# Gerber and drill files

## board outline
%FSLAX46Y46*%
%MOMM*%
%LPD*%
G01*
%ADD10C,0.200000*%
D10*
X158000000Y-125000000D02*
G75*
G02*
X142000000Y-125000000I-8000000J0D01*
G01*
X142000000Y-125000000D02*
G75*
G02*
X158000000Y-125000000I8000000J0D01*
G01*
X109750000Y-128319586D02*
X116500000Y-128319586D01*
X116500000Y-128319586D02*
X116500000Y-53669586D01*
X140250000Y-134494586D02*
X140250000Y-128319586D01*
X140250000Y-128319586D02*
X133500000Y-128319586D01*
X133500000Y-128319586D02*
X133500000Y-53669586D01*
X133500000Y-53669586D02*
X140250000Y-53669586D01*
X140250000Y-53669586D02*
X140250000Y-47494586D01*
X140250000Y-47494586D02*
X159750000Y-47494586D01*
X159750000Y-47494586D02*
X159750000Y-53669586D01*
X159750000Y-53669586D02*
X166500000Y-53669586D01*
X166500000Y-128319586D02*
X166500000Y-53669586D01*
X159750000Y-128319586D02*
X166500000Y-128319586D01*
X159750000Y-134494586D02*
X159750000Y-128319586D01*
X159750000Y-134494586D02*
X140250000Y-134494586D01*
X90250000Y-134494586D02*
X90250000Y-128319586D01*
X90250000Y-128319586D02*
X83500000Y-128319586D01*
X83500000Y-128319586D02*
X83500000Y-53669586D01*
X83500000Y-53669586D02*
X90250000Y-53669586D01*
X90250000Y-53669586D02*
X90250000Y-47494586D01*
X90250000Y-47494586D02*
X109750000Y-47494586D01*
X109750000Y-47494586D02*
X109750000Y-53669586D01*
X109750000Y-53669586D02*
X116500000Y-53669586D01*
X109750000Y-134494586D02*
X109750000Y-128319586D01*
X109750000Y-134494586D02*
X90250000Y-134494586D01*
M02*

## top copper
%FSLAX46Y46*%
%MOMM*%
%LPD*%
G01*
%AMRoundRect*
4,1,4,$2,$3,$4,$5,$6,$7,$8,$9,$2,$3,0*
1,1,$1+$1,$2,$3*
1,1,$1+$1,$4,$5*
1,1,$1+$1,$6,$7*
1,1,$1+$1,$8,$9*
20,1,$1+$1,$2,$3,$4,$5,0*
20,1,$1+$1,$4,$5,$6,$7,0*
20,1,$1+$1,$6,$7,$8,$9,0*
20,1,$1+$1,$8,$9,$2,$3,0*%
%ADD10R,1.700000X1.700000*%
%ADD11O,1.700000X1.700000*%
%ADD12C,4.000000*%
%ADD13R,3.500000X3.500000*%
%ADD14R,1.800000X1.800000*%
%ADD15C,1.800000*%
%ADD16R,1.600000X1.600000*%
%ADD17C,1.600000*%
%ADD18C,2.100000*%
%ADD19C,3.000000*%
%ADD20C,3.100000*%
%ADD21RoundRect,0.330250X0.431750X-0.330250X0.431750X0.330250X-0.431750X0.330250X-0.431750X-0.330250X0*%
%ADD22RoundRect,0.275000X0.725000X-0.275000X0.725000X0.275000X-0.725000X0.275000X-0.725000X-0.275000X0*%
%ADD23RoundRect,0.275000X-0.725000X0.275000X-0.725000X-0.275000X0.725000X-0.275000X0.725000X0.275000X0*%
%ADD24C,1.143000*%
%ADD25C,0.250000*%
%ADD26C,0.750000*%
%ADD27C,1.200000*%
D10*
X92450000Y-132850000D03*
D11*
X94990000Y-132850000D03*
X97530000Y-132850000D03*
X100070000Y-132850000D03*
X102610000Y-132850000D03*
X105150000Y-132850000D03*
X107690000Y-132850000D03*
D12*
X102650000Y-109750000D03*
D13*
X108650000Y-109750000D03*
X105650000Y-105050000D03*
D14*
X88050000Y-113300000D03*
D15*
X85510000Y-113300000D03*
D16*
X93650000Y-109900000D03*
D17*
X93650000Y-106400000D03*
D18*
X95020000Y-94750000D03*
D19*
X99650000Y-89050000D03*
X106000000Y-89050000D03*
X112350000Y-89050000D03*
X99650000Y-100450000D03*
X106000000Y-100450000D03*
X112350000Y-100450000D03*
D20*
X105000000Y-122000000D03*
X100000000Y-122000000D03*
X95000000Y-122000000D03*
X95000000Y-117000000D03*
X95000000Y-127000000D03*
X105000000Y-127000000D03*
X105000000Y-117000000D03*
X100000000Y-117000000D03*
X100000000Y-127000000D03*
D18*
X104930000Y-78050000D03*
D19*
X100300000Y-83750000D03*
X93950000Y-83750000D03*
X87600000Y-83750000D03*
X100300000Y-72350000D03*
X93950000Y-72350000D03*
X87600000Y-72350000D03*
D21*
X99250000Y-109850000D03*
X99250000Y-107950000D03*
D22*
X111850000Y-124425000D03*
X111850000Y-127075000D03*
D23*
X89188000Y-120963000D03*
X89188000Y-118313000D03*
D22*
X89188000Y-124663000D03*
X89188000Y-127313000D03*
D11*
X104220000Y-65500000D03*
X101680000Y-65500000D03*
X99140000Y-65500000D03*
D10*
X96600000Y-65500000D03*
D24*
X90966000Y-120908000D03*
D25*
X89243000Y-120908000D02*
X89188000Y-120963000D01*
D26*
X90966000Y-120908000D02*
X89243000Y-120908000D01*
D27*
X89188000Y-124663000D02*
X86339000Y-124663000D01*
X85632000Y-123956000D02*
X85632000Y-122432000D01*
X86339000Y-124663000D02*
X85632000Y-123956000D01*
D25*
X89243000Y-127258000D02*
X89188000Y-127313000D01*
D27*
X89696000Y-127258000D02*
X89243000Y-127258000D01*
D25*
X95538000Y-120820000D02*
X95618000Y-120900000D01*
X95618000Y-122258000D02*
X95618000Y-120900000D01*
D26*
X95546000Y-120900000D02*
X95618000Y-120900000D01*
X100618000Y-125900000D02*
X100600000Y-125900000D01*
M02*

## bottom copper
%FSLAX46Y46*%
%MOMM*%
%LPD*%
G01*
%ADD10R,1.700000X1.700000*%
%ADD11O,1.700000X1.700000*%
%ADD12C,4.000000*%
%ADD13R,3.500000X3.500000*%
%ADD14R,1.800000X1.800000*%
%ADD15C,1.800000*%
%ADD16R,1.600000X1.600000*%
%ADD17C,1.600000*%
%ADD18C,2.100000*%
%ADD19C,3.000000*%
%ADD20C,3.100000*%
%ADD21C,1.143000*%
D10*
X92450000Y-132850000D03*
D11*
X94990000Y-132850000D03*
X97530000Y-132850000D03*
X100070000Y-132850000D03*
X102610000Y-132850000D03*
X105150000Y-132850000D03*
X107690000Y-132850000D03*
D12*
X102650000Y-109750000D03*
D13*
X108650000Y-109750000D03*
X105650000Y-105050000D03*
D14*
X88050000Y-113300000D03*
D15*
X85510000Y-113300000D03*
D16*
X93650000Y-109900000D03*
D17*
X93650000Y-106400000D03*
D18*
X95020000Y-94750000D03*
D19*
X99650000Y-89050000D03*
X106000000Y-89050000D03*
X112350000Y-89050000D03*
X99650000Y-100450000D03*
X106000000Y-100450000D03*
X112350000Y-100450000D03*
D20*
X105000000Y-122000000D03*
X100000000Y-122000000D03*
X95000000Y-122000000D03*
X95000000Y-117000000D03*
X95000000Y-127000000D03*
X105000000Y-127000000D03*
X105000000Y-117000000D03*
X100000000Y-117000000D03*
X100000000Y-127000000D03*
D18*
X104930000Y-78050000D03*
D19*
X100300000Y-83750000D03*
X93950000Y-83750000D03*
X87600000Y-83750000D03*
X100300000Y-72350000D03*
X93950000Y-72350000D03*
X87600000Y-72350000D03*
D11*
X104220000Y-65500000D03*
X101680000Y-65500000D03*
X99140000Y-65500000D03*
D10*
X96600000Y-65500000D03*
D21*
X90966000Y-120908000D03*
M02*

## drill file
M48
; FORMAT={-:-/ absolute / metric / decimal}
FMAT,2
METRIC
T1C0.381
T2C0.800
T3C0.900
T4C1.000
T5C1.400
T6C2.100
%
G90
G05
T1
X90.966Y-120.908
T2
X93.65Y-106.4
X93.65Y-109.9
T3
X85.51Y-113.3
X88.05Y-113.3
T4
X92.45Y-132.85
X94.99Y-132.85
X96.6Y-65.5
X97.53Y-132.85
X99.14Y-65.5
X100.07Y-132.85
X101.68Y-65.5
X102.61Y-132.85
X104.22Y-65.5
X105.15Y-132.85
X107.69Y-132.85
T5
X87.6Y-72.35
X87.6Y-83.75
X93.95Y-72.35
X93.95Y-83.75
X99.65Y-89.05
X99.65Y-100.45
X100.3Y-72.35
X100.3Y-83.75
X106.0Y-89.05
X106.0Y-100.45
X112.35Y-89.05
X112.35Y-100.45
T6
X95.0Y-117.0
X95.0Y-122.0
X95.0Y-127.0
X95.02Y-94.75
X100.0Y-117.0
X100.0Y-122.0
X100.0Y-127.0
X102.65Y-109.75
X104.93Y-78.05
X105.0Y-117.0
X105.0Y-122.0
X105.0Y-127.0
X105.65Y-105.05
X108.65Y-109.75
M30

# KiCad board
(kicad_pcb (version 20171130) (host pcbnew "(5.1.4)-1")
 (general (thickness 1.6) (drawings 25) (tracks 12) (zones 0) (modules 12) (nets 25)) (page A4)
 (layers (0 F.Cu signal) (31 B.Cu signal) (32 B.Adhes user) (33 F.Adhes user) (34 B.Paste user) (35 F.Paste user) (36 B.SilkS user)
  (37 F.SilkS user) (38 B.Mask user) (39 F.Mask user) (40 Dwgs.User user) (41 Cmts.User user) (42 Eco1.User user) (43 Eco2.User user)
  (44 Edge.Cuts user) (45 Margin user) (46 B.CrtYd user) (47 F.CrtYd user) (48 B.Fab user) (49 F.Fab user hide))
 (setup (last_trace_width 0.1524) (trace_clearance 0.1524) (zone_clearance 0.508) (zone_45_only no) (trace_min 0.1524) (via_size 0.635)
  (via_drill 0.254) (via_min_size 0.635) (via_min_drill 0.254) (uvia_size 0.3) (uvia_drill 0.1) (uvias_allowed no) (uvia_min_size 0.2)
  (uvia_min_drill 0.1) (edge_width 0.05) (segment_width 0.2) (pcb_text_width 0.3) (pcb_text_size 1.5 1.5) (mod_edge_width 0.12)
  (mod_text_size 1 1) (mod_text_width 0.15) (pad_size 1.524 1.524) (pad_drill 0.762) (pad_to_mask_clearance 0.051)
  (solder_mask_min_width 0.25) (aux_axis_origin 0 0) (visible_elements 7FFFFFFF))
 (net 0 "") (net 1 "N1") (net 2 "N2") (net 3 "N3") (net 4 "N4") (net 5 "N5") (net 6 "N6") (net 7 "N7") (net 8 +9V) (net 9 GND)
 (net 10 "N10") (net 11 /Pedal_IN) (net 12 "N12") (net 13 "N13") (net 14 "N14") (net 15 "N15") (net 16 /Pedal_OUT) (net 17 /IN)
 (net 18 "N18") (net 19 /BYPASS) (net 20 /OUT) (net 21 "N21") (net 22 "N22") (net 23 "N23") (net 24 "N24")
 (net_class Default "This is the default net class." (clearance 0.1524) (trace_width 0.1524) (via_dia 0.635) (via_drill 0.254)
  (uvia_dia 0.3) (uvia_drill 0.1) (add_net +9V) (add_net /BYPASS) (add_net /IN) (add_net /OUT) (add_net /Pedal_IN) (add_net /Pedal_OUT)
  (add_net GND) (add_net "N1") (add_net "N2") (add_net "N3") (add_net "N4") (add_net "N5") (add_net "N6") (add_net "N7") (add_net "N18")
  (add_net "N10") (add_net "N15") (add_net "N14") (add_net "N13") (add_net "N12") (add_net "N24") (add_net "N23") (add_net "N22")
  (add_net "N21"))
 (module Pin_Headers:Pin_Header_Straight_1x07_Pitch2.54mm (layer F.Cu) (at 92.45 132.85 90)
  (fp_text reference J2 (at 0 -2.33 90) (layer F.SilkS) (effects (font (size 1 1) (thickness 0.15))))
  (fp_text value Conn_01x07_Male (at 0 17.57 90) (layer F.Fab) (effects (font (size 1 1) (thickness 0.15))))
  (pad 1 thru_hole rect (at 0 0 90) (size 1.7 1.7) (drill 1) (layers *.Cu *.Mask) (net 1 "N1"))
  (pad 2 thru_hole oval (at 0 2.54 90) (size 1.7 1.7) (drill 1) (layers *.Cu *.Mask) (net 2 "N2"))
  (pad 3 thru_hole oval (at 0 5.08 90) (size 1.7 1.7) (drill 1) (layers *.Cu *.Mask) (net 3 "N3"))
  (pad 4 thru_hole oval (at 0 7.62 90) (size 1.7 1.7) (drill 1) (layers *.Cu *.Mask) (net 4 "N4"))
  (pad 5 thru_hole oval (at 0 10.16 90) (size 1.7 1.7) (drill 1) (layers *.Cu *.Mask) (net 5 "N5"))
  (pad 6 thru_hole oval (at 0 12.7 90) (size 1.7 1.7) (drill 1) (layers *.Cu *.Mask) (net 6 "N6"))
  (pad 7 thru_hole oval (at 0 15.24 90) (size 1.7 1.7) (drill 1) (layers *.Cu *.Mask) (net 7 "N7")))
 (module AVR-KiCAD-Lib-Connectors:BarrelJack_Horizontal (layer F.Cu) (at 102.65 109.75 180)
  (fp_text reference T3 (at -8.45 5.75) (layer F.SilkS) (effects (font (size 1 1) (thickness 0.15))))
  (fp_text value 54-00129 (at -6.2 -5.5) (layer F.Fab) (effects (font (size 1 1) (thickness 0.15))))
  (pad 1 thru_hole circle (at 0 0 180) (size 4 4) (drill 2.1) (layers *.Cu *.Mask) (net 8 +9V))
  (pad 2 thru_hole rect (at -6 0 180) (size 3.5 3.5) (drill 2.1) (layers *.Cu *.Mask) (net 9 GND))
  (pad 3 thru_hole rect (at -3 4.7 180) (size 3.5 3.5) (drill 2.1) (layers *.Cu *.Mask) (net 9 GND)))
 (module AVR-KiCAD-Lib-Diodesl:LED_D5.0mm (layer F.Cu) (at 88.05 113.3 180)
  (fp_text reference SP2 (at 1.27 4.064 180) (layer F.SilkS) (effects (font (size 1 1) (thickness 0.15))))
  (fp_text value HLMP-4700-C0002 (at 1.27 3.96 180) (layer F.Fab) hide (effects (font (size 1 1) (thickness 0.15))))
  (pad 1 thru_hole rect (at 0 0 180) (size 1.8 1.8) (drill 0.9) (layers *.Cu *.Mask) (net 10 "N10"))
  (pad 2 thru_hole circle (at 2.54 0 180) (size 1.8 1.8) (drill 0.9) (layers *.Cu *.Mask) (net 8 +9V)))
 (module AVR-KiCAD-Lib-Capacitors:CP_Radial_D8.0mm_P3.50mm (layer F.Cu) (at 93.65 109.9 90)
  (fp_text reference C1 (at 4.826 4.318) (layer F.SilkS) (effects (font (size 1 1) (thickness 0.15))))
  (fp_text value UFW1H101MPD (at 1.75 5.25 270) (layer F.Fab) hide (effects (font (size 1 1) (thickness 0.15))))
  (pad 1 thru_hole rect (at 0 0 90) (size 1.6 1.6) (drill 0.8) (layers *.Cu *.Mask) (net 8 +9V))
  (pad 2 thru_hole circle (at 3.5 0 90) (size 1.6 1.6) (drill 0.8) (layers *.Cu *.Mask) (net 9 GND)))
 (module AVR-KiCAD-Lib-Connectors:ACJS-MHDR (layer F.Cu) (at 106 94.75)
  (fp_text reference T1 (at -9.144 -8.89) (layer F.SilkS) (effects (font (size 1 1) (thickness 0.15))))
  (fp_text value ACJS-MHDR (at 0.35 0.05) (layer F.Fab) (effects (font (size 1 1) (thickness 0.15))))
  (pad 7 thru_hole circle (at -10.98 0) (size 2.1 2.1) (drill 2.1) (layers *.Cu *.Mask))
  (pad 6 thru_hole circle (at -6.35 -5.7) (size 3 3) (drill 1.4) (layers *.Cu *.Mask) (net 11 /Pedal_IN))
  (pad 5 thru_hole circle (at 0 -5.7) (size 3 3) (drill 1.4) (layers *.Cu *.Mask) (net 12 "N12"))
  (pad 4 thru_hole circle (at 6.35 -5.7) (size 3 3) (drill 1.4) (layers *.Cu *.Mask) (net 9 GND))
  (pad 3 thru_hole circle (at -6.35 5.7) (size 3 3) (drill 1.4) (layers *.Cu *.Mask) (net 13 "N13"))
  (pad 2 thru_hole circle (at 0 5.7) (size 3 3) (drill 1.4) (layers *.Cu *.Mask) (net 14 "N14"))
  (pad 1 thru_hole circle (at 6.35 5.7) (size 3 3) (drill 1.4) (layers *.Cu *.Mask) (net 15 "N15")))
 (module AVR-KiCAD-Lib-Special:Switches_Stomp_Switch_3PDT (layer F.Cu) (at 100 122)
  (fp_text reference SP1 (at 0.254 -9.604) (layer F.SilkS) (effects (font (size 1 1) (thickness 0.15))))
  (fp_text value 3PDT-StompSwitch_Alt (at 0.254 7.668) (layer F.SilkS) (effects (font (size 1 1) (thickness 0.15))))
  (pad 4 thru_hole circle (at 5 0) (size 3.1 3.1) (drill 2.1) (layers *.Cu *.Mask F.SilkS) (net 11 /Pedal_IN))
  (pad 5 thru_hole circle (at 0 0) (size 3.1 3.1) (drill 2.1) (layers *.Cu *.Mask F.SilkS) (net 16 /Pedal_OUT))
  (pad 6 thru_hole circle (at -5 0) (size 3.1 3.1) (drill 2.1) (layers *.Cu *.Mask F.SilkS) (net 9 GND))
  (pad 3 thru_hole circle (at -5 -5) (size 3.1 3.1) (drill 2.1) (layers *.Cu *.Mask F.SilkS) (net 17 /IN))
  (pad 9 thru_hole circle (at -5 5) (size 3.1 3.1) (drill 2.1) (layers *.Cu *.Mask F.SilkS) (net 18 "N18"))
  (pad 7 thru_hole circle (at 5 5) (size 3.1 3.1) (drill 2.1) (layers *.Cu *.Mask F.SilkS) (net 17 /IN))
  (pad 1 thru_hole circle (at 5 -5) (size 3.1 3.1) (drill 2.1) (layers *.Cu *.Mask F.SilkS) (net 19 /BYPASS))
  (pad 2 thru_hole circle (at 0 -5) (size 3.1 3.1) (drill 2.1) (layers *.Cu *.Mask F.SilkS) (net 19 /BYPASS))
  (pad 8 thru_hole circle (at 0 5) (size 3.1 3.1) (drill 2.1) (layers *.Cu *.Mask F.SilkS) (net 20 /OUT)))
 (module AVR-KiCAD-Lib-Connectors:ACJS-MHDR (layer F.Cu) (at 93.95 78.05 180)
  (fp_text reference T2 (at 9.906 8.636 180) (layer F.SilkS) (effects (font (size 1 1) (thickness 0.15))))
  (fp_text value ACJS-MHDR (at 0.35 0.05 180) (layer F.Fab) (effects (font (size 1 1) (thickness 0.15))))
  (pad 7 thru_hole circle (at -10.98 0 180) (size 2.1 2.1) (drill 2.1) (layers *.Cu *.Mask))
  (pad 6 thru_hole circle (at -6.35 -5.7 180) (size 3 3) (drill 1.4) (layers *.Cu *.Mask) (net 16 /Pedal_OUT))
  (pad 5 thru_hole circle (at 0 -5.7 180) (size 3 3) (drill 1.4) (layers *.Cu *.Mask) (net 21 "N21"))
  (pad 4 thru_hole circle (at 6.35 -5.7 180) (size 3 3) (drill 1.4) (layers *.Cu *.Mask) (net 9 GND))
  (pad 3 thru_hole circle (at -6.35 5.7 180) (size 3 3) (drill 1.4) (layers *.Cu *.Mask) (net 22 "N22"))
  (pad 2 thru_hole circle (at 0 5.7 180) (size 3 3) (drill 1.4) (layers *.Cu *.Mask) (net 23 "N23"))
  (pad 1 thru_hole circle (at 6.35 5.7 180) (size 3 3) (drill 1.4) (layers *.Cu *.Mask) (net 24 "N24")))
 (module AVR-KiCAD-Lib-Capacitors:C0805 (layer F.Cu) (at 99.25 108.9 90)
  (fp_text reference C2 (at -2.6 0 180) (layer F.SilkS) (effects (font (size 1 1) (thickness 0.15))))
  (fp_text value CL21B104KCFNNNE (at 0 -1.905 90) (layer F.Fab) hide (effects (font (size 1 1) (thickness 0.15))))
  (pad 1 smd roundrect (at -0.95 0 90) (size 1.321 1.524) (layers F.Cu F.Paste F.Mask) (roundrect_rratio 0.25) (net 8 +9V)
   (solder_mask_margin 0.102))
  (pad 2 smd roundrect (at 0.95 0 90) (size 1.321 1.524) (layers F.Cu F.Paste F.Mask) (roundrect_rratio 0.25) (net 9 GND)
   (solder_mask_margin 0.102)))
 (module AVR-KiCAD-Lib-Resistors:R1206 (layer F.Cu) (at 111.85 125.75 90)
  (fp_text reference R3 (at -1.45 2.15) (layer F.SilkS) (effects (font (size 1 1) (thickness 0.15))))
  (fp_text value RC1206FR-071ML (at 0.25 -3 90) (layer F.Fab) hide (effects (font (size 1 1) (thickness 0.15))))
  (pad 2 smd roundrect (at 1.325 0 90) (size 1.1 2) (layers F.Cu F.Paste F.Mask) (roundrect_rratio 0.25) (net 9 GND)
   (solder_mask_margin 0.102))
  (pad 1 smd roundrect (at -1.325 0 90) (size 1.1 2) (layers F.Cu F.Paste F.Mask) (roundrect_rratio 0.25) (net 20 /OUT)
   (solder_mask_margin 0.102)))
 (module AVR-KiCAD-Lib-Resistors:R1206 (layer F.Cu) (at 89.188 119.638 270)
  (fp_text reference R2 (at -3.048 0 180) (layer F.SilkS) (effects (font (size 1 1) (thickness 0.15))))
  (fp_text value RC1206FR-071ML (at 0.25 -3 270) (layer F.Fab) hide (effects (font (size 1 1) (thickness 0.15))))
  (pad 2 smd roundrect (at 1.325 0 270) (size 1.1 2) (layers F.Cu F.Paste F.Mask) (roundrect_rratio 0.25) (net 9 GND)
   (solder_mask_margin 0.102))
  (pad 1 smd roundrect (at -1.325 0 270) (size 1.1 2) (layers F.Cu F.Paste F.Mask) (roundrect_rratio 0.25) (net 17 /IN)
   (solder_mask_margin 0.102)))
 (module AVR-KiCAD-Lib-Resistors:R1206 (layer F.Cu) (at 89.188 125.988 90)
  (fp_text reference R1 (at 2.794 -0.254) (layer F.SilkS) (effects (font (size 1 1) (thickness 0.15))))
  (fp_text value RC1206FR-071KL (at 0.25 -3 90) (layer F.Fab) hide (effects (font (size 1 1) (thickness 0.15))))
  (pad 2 smd roundrect (at 1.325 0 90) (size 1.1 2) (layers F.Cu F.Paste F.Mask) (roundrect_rratio 0.25) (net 10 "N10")
   (solder_mask_margin 0.102))
  (pad 1 smd roundrect (at -1.325 0 90) (size 1.1 2) (layers F.Cu F.Paste F.Mask) (roundrect_rratio 0.25) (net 18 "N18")
   (solder_mask_margin 0.102)))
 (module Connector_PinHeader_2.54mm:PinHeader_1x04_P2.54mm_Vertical (layer F.Cu) (at 96.6 65.5 90)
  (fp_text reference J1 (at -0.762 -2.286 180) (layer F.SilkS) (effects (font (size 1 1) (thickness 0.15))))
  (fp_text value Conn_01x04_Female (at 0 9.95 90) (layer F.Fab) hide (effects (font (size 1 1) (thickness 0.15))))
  (pad 4 thru_hole oval (at 0 7.62 90) (size 1.7 1.7) (drill 1) (layers *.Cu *.Mask) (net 20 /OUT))
  (pad 3 thru_hole oval (at 0 5.08 90) (size 1.7 1.7) (drill 1) (layers *.Cu *.Mask) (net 8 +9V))
  (pad 2 thru_hole oval (at 0 2.54 90) (size 1.7 1.7) (drill 1) (layers *.Cu *.Mask) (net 9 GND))
  (pad 1 thru_hole rect (at 0 0 90) (size 1.7 1.7) (drill 1) (layers *.Cu *.Mask) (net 17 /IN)))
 (gr_circle (center 150 125) (end 158 125) (layer Edge.Cuts) (width 0.2))
 (gr_line (start 109.75 128.319586) (end 116.5 128.319586) (layer Edge.Cuts) (width 0.2))
 (gr_line (start 116.5 128.319586) (end 116.5 53.669586) (layer Edge.Cuts) (width 0.2))
 (gr_line (start 140.25 134.494586) (end 140.25 128.319586) (layer Edge.Cuts) (width 0.2))
 (gr_line (start 140.25 128.319586) (end 133.5 128.319586) (layer Edge.Cuts) (width 0.2))
 (gr_line (start 133.5 128.319586) (end 133.5 53.669586) (layer Edge.Cuts) (width 0.2))
 (gr_line (start 133.5 53.669586) (end 140.25 53.669586) (layer Edge.Cuts) (width 0.2))
 (gr_line (start 140.25 53.669586) (end 140.25 47.494586) (layer Edge.Cuts) (width 0.2))
 (gr_line (start 140.25 47.494586) (end 159.75 47.494586) (layer Edge.Cuts) (width 0.2))
 (gr_line (start 159.75 47.494586) (end 159.75 53.669586) (layer Edge.Cuts) (width 0.2))
 (gr_line (start 159.75 53.669586) (end 166.5 53.669586) (layer Edge.Cuts) (width 0.2))
 (gr_line (start 166.5 128.319586) (end 166.5 53.669586) (layer Edge.Cuts) (width 0.2))
 (gr_line (start 159.75 128.319586) (end 166.5 128.319586) (layer Edge.Cuts) (width 0.2))
 (gr_line (start 159.75 134.494586) (end 159.75 128.319586) (layer Edge.Cuts) (width 0.2))
 (gr_line (start 159.75 134.494586) (end 140.25 134.494586) (layer Edge.Cuts) (width 0.2))
 (gr_line (start 90.25 134.494586) (end 90.25 128.319586) (layer Edge.Cuts) (width 0.2))
 (gr_line (start 90.25 128.319586) (end 83.5 128.319586) (layer Edge.Cuts) (width 0.2))
 (gr_line (start 83.5 128.319586) (end 83.5 53.669586) (layer Edge.Cuts) (width 0.2))
 (gr_line (start 83.5 53.669586) (end 90.25 53.669586) (layer Edge.Cuts) (width 0.2))
 (gr_line (start 90.25 53.669586) (end 90.25 47.494586) (layer Edge.Cuts) (width 0.2))
 (gr_line (start 90.25 47.494586) (end 109.75 47.494586) (layer Edge.Cuts) (width 0.2))
 (gr_line (start 109.75 47.494586) (end 109.75 53.669586) (layer Edge.Cuts) (width 0.2))
 (gr_line (start 109.75 53.669586) (end 116.5 53.669586) (layer Edge.Cuts) (width 0.2))
 (gr_line (start 109.75 134.494586) (end 109.75 128.319586) (layer Edge.Cuts) (width 0.2))
 (gr_line (start 109.75 134.494586) (end 90.25 134.494586) (layer Edge.Cuts) (width 0.2))
 (via (at 90.966 120.908) (size 1.143) (drill 0.381) (layers F.Cu B.Cu) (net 9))
 (segment (start 89.243 120.908) (end 89.188 120.963) (width 0.25) (layer F.Cu) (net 9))
 (segment (start 90.966 120.908) (end 89.243 120.908) (width 0.75) (layer F.Cu) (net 9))
 (segment (start 89.188 124.663) (end 86.339 124.663) (width 1.2) (layer F.Cu) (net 10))
 (segment (start 85.632 123.956) (end 85.632 122.432) (width 1.2) (layer F.Cu) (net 10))
 (segment (start 86.339 124.663) (end 85.632 123.956) (width 1.2) (layer F.Cu) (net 10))
 (segment (start 89.243 127.258) (end 89.188 127.313) (width 0.25) (layer F.Cu) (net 18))
 (segment (start 89.696 127.258) (end 89.243 127.258) (width 1.2) (layer F.Cu) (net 18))
 (segment (start 95.538 120.82) (end 95.618 120.9) (width 0.25) (layer F.Cu) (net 9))
 (segment (start 95.618 122.258) (end 95.618 120.9) (width 0.25) (layer F.Cu) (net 9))
 (segment (start 95.546 120.9) (end 95.618 120.9) (width 0.75) (layer F.Cu) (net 9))
 (segment (start 100.618 125.9) (end 100.6 125.9) (width 0.75) (layer F.Cu) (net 20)))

